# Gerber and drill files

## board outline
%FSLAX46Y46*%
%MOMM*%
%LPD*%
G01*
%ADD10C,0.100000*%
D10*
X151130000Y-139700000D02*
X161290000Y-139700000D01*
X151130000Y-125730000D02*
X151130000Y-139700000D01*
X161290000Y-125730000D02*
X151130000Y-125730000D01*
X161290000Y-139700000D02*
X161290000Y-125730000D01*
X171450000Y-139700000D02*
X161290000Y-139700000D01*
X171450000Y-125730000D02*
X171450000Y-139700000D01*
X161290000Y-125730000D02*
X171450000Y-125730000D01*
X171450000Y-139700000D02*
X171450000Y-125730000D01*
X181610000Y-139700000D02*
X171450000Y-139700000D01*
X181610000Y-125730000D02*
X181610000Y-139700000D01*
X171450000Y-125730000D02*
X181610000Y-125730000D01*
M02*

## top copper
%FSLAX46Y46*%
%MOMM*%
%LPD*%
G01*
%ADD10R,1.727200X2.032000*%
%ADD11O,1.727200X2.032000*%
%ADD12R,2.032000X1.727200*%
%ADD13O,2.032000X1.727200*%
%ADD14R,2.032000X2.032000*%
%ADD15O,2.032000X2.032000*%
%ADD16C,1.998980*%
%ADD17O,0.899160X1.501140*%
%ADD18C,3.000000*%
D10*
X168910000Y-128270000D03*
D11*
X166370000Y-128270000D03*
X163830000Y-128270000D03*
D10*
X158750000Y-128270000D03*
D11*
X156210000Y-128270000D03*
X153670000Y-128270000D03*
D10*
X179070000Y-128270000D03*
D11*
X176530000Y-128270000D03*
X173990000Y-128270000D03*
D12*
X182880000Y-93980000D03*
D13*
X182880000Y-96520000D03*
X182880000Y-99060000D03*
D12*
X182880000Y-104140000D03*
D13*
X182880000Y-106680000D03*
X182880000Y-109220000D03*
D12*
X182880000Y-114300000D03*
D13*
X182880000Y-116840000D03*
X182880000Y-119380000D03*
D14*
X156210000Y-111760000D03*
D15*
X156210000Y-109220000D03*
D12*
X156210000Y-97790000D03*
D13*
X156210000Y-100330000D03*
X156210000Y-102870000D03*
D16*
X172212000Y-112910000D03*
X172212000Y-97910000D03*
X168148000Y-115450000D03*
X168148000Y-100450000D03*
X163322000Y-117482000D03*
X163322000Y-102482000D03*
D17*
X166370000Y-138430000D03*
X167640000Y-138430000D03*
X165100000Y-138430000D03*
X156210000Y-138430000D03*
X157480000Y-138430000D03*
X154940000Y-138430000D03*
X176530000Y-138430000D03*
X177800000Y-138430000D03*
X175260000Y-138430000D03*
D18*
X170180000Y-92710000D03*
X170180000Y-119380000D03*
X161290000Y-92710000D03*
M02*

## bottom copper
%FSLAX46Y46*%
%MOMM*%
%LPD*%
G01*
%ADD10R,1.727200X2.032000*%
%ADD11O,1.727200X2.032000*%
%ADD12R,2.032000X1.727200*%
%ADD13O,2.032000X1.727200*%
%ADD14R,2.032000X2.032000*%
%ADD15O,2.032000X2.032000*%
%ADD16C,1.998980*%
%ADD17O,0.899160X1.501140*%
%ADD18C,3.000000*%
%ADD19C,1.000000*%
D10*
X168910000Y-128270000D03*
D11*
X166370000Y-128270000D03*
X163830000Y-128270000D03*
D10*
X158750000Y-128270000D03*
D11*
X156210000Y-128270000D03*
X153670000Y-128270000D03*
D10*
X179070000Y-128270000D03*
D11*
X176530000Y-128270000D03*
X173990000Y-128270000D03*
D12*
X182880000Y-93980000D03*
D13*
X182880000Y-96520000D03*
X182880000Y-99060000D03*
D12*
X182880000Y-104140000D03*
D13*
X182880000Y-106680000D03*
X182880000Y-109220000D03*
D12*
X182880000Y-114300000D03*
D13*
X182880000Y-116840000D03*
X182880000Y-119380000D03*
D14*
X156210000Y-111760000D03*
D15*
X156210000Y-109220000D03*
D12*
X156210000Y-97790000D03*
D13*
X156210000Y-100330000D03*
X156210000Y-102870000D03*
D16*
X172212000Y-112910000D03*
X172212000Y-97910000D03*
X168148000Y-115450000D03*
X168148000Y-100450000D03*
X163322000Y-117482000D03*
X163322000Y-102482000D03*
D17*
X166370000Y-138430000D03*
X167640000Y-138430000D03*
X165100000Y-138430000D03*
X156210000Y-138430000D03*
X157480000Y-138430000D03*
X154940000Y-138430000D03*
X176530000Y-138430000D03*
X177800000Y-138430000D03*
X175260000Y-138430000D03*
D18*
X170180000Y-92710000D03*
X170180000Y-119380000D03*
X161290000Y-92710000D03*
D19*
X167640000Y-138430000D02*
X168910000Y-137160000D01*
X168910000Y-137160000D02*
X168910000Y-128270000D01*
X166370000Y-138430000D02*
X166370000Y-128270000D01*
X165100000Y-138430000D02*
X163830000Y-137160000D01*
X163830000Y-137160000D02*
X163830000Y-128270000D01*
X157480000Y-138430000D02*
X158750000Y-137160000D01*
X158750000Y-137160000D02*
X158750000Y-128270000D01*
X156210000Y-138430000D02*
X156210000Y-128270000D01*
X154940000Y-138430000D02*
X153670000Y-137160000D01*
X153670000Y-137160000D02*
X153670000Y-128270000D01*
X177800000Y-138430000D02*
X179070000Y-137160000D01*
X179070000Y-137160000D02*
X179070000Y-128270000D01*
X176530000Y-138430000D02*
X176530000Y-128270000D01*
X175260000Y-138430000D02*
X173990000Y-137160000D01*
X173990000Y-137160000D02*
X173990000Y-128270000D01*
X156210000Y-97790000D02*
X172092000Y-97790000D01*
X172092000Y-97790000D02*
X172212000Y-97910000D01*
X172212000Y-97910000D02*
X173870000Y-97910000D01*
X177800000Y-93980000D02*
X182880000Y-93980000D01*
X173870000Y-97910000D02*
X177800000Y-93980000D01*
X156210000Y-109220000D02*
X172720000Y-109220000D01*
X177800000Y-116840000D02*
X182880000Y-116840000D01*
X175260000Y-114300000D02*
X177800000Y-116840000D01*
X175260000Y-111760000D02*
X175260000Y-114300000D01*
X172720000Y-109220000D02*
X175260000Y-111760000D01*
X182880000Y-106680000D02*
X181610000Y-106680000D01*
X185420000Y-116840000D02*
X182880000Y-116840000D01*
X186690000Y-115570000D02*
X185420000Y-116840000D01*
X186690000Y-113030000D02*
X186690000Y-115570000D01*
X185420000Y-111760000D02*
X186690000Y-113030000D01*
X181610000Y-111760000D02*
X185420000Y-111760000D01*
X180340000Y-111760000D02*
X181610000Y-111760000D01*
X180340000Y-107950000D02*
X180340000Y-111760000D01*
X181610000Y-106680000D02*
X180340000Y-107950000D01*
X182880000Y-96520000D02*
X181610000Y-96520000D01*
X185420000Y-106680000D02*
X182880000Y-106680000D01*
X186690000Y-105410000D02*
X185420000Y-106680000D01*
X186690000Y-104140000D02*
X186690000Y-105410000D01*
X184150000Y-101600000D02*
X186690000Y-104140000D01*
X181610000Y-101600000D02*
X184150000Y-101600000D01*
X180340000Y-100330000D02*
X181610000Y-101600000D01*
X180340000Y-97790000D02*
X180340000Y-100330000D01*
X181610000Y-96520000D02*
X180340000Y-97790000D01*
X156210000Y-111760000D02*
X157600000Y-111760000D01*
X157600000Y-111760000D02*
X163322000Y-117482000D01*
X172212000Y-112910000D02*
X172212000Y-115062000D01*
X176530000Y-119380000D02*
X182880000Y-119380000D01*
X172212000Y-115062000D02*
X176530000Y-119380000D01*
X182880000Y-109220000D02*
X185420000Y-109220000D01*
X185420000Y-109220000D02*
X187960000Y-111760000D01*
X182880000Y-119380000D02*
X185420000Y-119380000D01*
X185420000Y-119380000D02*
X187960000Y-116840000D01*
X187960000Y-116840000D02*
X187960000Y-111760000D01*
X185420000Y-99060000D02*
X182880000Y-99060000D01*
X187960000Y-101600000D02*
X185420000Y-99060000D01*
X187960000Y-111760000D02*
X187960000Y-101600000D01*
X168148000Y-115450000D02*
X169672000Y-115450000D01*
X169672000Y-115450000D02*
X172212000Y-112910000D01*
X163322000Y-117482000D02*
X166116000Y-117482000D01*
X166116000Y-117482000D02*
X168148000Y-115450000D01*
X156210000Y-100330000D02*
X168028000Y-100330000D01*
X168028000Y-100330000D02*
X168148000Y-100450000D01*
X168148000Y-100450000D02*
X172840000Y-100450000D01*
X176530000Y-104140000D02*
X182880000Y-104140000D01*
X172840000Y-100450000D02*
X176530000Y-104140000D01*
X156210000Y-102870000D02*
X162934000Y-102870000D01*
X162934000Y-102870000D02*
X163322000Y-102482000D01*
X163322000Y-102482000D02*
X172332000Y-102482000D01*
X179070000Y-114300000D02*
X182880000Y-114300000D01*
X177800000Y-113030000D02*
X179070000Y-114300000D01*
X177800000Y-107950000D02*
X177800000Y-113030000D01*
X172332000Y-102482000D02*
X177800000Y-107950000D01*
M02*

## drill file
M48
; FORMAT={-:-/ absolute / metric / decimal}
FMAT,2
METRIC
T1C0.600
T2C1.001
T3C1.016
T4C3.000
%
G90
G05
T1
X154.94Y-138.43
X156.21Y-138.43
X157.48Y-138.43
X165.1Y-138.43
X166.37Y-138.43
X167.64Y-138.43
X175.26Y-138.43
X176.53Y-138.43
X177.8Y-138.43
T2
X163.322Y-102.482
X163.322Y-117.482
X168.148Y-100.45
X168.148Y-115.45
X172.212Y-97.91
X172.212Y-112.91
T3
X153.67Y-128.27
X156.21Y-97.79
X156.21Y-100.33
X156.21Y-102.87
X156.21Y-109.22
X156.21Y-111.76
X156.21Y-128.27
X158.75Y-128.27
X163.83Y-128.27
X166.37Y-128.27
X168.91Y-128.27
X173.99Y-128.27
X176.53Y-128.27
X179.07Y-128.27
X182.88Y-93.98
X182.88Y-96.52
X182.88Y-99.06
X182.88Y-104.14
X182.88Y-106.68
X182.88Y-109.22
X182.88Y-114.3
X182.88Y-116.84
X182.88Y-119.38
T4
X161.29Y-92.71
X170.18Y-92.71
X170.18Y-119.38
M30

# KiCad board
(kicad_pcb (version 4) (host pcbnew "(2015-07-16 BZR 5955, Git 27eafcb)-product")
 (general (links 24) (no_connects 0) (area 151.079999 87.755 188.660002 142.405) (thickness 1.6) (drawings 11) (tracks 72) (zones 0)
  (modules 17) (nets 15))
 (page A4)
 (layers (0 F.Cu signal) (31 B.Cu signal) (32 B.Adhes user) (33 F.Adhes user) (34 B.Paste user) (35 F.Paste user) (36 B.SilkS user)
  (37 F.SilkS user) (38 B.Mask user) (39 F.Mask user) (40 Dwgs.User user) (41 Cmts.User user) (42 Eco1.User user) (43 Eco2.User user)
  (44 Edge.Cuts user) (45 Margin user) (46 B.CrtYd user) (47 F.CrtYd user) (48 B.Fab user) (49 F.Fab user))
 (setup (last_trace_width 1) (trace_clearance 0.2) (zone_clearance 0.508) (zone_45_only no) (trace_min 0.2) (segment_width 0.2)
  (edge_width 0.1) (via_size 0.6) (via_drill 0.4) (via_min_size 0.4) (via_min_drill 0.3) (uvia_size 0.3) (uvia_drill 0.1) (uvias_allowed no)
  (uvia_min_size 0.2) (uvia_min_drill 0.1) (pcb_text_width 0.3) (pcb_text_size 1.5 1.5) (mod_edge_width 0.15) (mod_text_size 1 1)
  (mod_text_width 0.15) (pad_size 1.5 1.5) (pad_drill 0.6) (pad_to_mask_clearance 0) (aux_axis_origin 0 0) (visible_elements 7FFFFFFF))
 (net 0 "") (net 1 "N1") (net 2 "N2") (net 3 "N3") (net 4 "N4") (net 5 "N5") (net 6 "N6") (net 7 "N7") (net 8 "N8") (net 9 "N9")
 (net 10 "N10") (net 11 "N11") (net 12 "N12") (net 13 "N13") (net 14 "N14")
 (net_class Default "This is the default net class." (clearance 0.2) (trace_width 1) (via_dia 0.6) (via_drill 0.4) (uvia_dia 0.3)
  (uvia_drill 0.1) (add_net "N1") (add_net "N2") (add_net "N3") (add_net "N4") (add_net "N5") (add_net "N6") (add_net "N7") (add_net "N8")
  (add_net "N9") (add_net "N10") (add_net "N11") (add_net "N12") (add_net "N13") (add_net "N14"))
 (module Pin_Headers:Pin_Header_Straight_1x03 (layer F.Cu) (at 168.91 128.27 270)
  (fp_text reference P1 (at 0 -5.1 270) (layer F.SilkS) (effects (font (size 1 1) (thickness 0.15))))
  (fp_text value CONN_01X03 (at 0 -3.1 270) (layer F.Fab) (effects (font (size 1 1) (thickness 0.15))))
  (pad 1 thru_hole rect (at 0 0 270) (size 2.032 1.7272) (drill 1.016) (layers *.Cu *.Mask F.SilkS) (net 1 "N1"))
  (pad 2 thru_hole oval (at 0 2.54 270) (size 2.032 1.7272) (drill 1.016) (layers *.Cu *.Mask F.SilkS) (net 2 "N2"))
  (pad 3 thru_hole oval (at 0 5.08 270) (size 2.032 1.7272) (drill 1.016) (layers *.Cu *.Mask F.SilkS) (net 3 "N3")))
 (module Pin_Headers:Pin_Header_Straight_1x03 (layer F.Cu) (at 158.75 128.27 270)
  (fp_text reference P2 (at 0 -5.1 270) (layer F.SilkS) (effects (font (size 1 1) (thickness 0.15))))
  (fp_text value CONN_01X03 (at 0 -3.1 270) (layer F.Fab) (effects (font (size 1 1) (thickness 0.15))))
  (pad 1 thru_hole rect (at 0 0 270) (size 2.032 1.7272) (drill 1.016) (layers *.Cu *.Mask F.SilkS) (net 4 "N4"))
  (pad 2 thru_hole oval (at 0 2.54 270) (size 2.032 1.7272) (drill 1.016) (layers *.Cu *.Mask F.SilkS) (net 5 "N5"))
  (pad 3 thru_hole oval (at 0 5.08 270) (size 2.032 1.7272) (drill 1.016) (layers *.Cu *.Mask F.SilkS) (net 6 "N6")))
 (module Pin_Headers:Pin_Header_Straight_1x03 (layer F.Cu) (at 179.07 128.27 270)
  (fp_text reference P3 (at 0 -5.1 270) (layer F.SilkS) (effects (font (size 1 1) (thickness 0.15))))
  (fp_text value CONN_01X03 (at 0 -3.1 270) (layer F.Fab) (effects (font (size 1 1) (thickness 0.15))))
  (pad 1 thru_hole rect (at 0 0 270) (size 2.032 1.7272) (drill 1.016) (layers *.Cu *.Mask F.SilkS) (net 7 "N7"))
  (pad 2 thru_hole oval (at 0 2.54 270) (size 2.032 1.7272) (drill 1.016) (layers *.Cu *.Mask F.SilkS) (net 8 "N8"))
  (pad 3 thru_hole oval (at 0 5.08 270) (size 2.032 1.7272) (drill 1.016) (layers *.Cu *.Mask F.SilkS) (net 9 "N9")))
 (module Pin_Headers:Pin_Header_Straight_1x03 (layer F.Cu) (at 182.88 93.98)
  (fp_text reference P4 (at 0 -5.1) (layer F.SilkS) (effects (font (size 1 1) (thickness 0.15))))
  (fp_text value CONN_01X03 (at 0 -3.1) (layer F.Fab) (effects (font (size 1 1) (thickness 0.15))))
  (pad 1 thru_hole rect (at 0 0) (size 2.032 1.7272) (drill 1.016) (layers *.Cu *.Mask F.SilkS) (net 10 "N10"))
  (pad 2 thru_hole oval (at 0 2.54) (size 2.032 1.7272) (drill 1.016) (layers *.Cu *.Mask F.SilkS) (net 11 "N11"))
  (pad 3 thru_hole oval (at 0 5.08) (size 2.032 1.7272) (drill 1.016) (layers *.Cu *.Mask F.SilkS) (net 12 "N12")))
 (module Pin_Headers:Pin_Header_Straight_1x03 (layer F.Cu) (at 182.88 104.14)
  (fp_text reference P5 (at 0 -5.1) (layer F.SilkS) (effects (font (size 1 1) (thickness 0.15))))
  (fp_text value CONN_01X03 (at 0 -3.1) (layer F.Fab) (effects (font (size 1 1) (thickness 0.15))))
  (pad 1 thru_hole rect (at 0 0) (size 2.032 1.7272) (drill 1.016) (layers *.Cu *.Mask F.SilkS) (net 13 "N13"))
  (pad 2 thru_hole oval (at 0 2.54) (size 2.032 1.7272) (drill 1.016) (layers *.Cu *.Mask F.SilkS) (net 11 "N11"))
  (pad 3 thru_hole oval (at 0 5.08) (size 2.032 1.7272) (drill 1.016) (layers *.Cu *.Mask F.SilkS) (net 12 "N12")))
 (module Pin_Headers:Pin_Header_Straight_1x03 (layer F.Cu) (at 182.88 114.3)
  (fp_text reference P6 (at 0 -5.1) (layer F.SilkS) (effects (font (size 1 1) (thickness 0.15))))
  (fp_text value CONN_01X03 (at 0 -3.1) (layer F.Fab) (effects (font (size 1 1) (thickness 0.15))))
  (pad 1 thru_hole rect (at 0 0) (size 2.032 1.7272) (drill 1.016) (layers *.Cu *.Mask F.SilkS) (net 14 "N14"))
  (pad 2 thru_hole oval (at 0 2.54) (size 2.032 1.7272) (drill 1.016) (layers *.Cu *.Mask F.SilkS) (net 11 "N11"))
  (pad 3 thru_hole oval (at 0 5.08) (size 2.032 1.7272) (drill 1.016) (layers *.Cu *.Mask F.SilkS) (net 12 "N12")))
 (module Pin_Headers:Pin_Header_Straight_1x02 (layer F.Cu) (at 156.21 111.76 180)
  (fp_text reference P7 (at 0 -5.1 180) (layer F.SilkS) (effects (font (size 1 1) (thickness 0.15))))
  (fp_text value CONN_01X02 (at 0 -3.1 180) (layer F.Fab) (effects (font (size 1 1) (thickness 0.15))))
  (pad 1 thru_hole rect (at 0 0 180) (size 2.032 2.032) (drill 1.016) (layers *.Cu *.Mask F.SilkS) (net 12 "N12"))
  (pad 2 thru_hole oval (at 0 2.54 180) (size 2.032 2.032) (drill 1.016) (layers *.Cu *.Mask F.SilkS) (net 11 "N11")))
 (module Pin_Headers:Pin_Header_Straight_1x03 (layer F.Cu) (at 156.21 97.79)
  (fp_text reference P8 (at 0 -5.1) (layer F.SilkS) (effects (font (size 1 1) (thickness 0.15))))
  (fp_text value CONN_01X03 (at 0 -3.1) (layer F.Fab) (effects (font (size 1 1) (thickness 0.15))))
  (pad 1 thru_hole rect (at 0 0) (size 2.032 1.7272) (drill 1.016) (layers *.Cu *.Mask F.SilkS) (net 10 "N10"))
  (pad 2 thru_hole oval (at 0 2.54) (size 2.032 1.7272) (drill 1.016) (layers *.Cu *.Mask F.SilkS) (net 13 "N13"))
  (pad 3 thru_hole oval (at 0 5.08) (size 2.032 1.7272) (drill 1.016) (layers *.Cu *.Mask F.SilkS) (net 14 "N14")))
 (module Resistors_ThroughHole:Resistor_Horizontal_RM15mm (layer F.Cu) (at 172.212 105.41 90)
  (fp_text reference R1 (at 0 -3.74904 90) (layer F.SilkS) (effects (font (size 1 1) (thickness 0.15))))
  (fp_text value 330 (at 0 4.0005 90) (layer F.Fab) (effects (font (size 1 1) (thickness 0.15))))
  (pad 1 thru_hole circle (at -7.5 0 90) (size 1.99898 1.99898) (drill 1.00076) (layers *.Cu *.SilkS *.Mask) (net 12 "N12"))
  (pad 2 thru_hole circle (at 7.5 0 90) (size 1.99898 1.99898) (drill 1.00076) (layers *.Cu *.SilkS *.Mask) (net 10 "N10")))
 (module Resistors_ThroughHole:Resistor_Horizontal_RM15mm (layer F.Cu) (at 168.148 107.95 90)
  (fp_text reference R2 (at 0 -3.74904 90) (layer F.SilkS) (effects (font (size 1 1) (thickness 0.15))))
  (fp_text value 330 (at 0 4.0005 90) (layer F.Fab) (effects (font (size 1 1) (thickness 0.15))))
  (pad 1 thru_hole circle (at -7.5 0 90) (size 1.99898 1.99898) (drill 1.00076) (layers *.Cu *.SilkS *.Mask) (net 12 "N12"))
  (pad 2 thru_hole circle (at 7.5 0 90) (size 1.99898 1.99898) (drill 1.00076) (layers *.Cu *.SilkS *.Mask) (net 13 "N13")))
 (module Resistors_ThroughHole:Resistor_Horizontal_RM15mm (layer F.Cu) (at 163.322 109.982 90)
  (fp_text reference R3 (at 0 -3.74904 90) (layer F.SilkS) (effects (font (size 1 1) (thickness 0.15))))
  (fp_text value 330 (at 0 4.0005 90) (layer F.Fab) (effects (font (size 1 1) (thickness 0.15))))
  (pad 1 thru_hole circle (at -7.5 0 90) (size 1.99898 1.99898) (drill 1.00076) (layers *.Cu *.SilkS *.Mask) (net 12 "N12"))
  (pad 2 thru_hole circle (at 7.5 0 90) (size 1.99898 1.99898) (drill 1.00076) (layers *.Cu *.SilkS *.Mask) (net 14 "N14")))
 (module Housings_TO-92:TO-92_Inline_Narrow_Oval (layer F.Cu) (at 165.1 138.43)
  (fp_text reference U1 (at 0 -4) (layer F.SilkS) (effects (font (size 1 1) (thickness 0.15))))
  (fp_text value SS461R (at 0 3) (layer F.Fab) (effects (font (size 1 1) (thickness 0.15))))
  (pad 2 thru_hole oval (at 1.27 0 180) (size 0.89916 1.50114) (drill 0.6) (layers *.Cu *.Mask F.SilkS) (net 2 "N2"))
  (pad 3 thru_hole oval (at 2.54 0 180) (size 0.89916 1.50114) (drill 0.6) (layers *.Cu *.Mask F.SilkS) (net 1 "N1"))
  (pad 1 thru_hole oval (at 0 0 180) (size 0.89916 1.50114) (drill 0.6) (layers *.Cu *.Mask F.SilkS) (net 3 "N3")))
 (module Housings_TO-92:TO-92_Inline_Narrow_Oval (layer F.Cu) (at 154.94 138.43)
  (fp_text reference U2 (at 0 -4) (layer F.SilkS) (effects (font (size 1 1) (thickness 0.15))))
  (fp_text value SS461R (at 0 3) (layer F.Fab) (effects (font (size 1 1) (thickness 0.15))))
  (pad 2 thru_hole oval (at 1.27 0 180) (size 0.89916 1.50114) (drill 0.6) (layers *.Cu *.Mask F.SilkS) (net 5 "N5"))
  (pad 3 thru_hole oval (at 2.54 0 180) (size 0.89916 1.50114) (drill 0.6) (layers *.Cu *.Mask F.SilkS) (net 4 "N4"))
  (pad 1 thru_hole oval (at 0 0 180) (size 0.89916 1.50114) (drill 0.6) (layers *.Cu *.Mask F.SilkS) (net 6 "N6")))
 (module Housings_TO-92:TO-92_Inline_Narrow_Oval (layer F.Cu) (at 175.26 138.43)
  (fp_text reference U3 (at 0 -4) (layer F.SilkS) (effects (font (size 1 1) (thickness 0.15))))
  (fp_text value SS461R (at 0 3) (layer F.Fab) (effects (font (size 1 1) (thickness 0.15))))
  (pad 2 thru_hole oval (at 1.27 0 180) (size 0.89916 1.50114) (drill 0.6) (layers *.Cu *.Mask F.SilkS) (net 8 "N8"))
  (pad 3 thru_hole oval (at 2.54 0 180) (size 0.89916 1.50114) (drill 0.6) (layers *.Cu *.Mask F.SilkS) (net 7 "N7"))
  (pad 1 thru_hole oval (at 0 0 180) (size 0.89916 1.50114) (drill 0.6) (layers *.Cu *.Mask F.SilkS) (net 9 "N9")))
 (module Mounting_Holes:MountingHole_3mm (layer F.Cu) (at 170.18 92.71)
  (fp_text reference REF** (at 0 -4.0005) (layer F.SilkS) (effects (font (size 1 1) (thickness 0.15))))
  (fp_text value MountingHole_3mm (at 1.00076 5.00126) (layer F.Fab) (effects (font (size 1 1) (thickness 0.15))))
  (pad 1 thru_hole circle (at 0 0) (size 3 3) (drill 3) (layers)))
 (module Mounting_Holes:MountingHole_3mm (layer F.Cu) (at 170.18 119.38)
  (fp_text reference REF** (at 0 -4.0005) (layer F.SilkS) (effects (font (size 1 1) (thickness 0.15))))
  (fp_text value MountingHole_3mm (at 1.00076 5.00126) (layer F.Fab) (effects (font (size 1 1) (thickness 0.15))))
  (pad 1 thru_hole circle (at 0 0) (size 3 3) (drill 3) (layers)))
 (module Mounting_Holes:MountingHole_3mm (layer F.Cu) (at 161.29 92.71)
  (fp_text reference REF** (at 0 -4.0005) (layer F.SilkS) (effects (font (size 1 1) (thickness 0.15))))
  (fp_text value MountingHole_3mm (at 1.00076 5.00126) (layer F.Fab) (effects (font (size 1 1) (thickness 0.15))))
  (pad 1 thru_hole circle (at 0 0) (size 3 3) (drill 3) (layers)))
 (gr_line (start 151.13 139.7) (end 161.29 139.7) (angle 90) (layer Edge.Cuts) (width 0.1))
 (gr_line (start 151.13 125.73) (end 151.13 139.7) (angle 90) (layer Edge.Cuts) (width 0.1))
 (gr_line (start 161.29 125.73) (end 151.13 125.73) (angle 90) (layer Edge.Cuts) (width 0.1))
 (gr_line (start 161.29 139.7) (end 161.29 125.73) (angle 90) (layer Edge.Cuts) (width 0.1))
 (gr_line (start 171.45 139.7) (end 161.29 139.7) (angle 90) (layer Edge.Cuts) (width 0.1))
 (gr_line (start 171.45 125.73) (end 171.45 139.7) (angle 90) (layer Edge.Cuts) (width 0.1))
 (gr_line (start 161.29 125.73) (end 171.45 125.73) (angle 90) (layer Edge.Cuts) (width 0.1))
 (gr_line (start 171.45 139.7) (end 171.45 125.73) (angle 90) (layer Edge.Cuts) (width 0.1))
 (gr_line (start 181.61 139.7) (end 171.45 139.7) (angle 90) (layer Edge.Cuts) (width 0.1))
 (gr_line (start 181.61 125.73) (end 181.61 139.7) (angle 90) (layer Edge.Cuts) (width 0.1))
 (gr_line (start 171.45 125.73) (end 181.61 125.73) (angle 90) (layer Edge.Cuts) (width 0.1))
 (segment (start 167.64 138.43) (end 168.91 137.16) (width 1) (layer B.Cu) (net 1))
 (segment (start 168.91 137.16) (end 168.91 128.27) (width 1) (layer B.Cu) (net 1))
 (segment (start 166.37 138.43) (end 166.37 128.27) (width 1) (layer B.Cu) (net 2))
 (segment (start 165.1 138.43) (end 163.83 137.16) (width 1) (layer B.Cu) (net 3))
 (segment (start 163.83 137.16) (end 163.83 128.27) (width 1) (layer B.Cu) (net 3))
 (segment (start 157.48 138.43) (end 158.75 137.16) (width 1) (layer B.Cu) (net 4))
 (segment (start 158.75 137.16) (end 158.75 128.27) (width 1) (layer B.Cu) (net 4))
 (segment (start 156.21 138.43) (end 156.21 128.27) (width 1) (layer B.Cu) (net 5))
 (segment (start 154.94 138.43) (end 153.67 137.16) (width 1) (layer B.Cu) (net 6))
 (segment (start 153.67 137.16) (end 153.67 128.27) (width 1) (layer B.Cu) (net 6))
 (segment (start 177.8 138.43) (end 179.07 137.16) (width 1) (layer B.Cu) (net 7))
 (segment (start 179.07 137.16) (end 179.07 128.27) (width 1) (layer B.Cu) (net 7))
 (segment (start 176.53 138.43) (end 176.53 128.27) (width 1) (layer B.Cu) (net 8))
 (segment (start 175.26 138.43) (end 173.99 137.16) (width 1) (layer B.Cu) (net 9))
 (segment (start 173.99 137.16) (end 173.99 128.27) (width 1) (layer B.Cu) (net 9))
 (segment (start 156.21 97.79) (end 172.092 97.79) (width 1) (layer B.Cu) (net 10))
 (segment (start 172.092 97.79) (end 172.212 97.91) (width 1) (layer B.Cu) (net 10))
 (segment (start 172.212 97.91) (end 173.87 97.91) (width 1) (layer B.Cu) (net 10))
 (segment (start 177.8 93.98) (end 182.88 93.98) (width 1) (layer B.Cu) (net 10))
 (segment (start 173.87 97.91) (end 177.8 93.98) (width 1) (layer B.Cu) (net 10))
 (segment (start 156.21 109.22) (end 172.72 109.22) (width 1) (layer B.Cu) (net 11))
 (segment (start 177.8 116.84) (end 182.88 116.84) (width 1) (layer B.Cu) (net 11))
 (segment (start 175.26 114.3) (end 177.8 116.84) (width 1) (layer B.Cu) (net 11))
 (segment (start 175.26 111.76) (end 175.26 114.3) (width 1) (layer B.Cu) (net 11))
 (segment (start 172.72 109.22) (end 175.26 111.76) (width 1) (layer B.Cu) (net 11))
 (segment (start 182.88 106.68) (end 181.61 106.68) (width 1) (layer B.Cu) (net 11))
 (segment (start 185.42 116.84) (end 182.88 116.84) (width 1) (layer B.Cu) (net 11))
 (segment (start 186.69 115.57) (end 185.42 116.84) (width 1) (layer B.Cu) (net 11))
 (segment (start 186.69 113.03) (end 186.69 115.57) (width 1) (layer B.Cu) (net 11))
 (segment (start 185.42 111.76) (end 186.69 113.03) (width 1) (layer B.Cu) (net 11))
 (segment (start 181.61 111.76) (end 185.42 111.76) (width 1) (layer B.Cu) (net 11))
 (segment (start 180.34 111.76) (end 181.61 111.76) (width 1) (layer B.Cu) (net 11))
 (segment (start 180.34 107.95) (end 180.34 111.76) (width 1) (layer B.Cu) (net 11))
 (segment (start 181.61 106.68) (end 180.34 107.95) (width 1) (layer B.Cu) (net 11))
 (segment (start 182.88 96.52) (end 181.61 96.52) (width 1) (layer B.Cu) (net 11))
 (segment (start 185.42 106.68) (end 182.88 106.68) (width 1) (layer B.Cu) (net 11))
 (segment (start 186.69 105.41) (end 185.42 106.68) (width 1) (layer B.Cu) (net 11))
 (segment (start 186.69 104.14) (end 186.69 105.41) (width 1) (layer B.Cu) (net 11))
 (segment (start 184.15 101.6) (end 186.69 104.14) (width 1) (layer B.Cu) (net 11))
 (segment (start 181.61 101.6) (end 184.15 101.6) (width 1) (layer B.Cu) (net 11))
 (segment (start 180.34 100.33) (end 181.61 101.6) (width 1) (layer B.Cu) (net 11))
 (segment (start 180.34 97.79) (end 180.34 100.33) (width 1) (layer B.Cu) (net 11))
 (segment (start 181.61 96.52) (end 180.34 97.79) (width 1) (layer B.Cu) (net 11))
 (segment (start 156.21 111.76) (end 157.6 111.76) (width 1) (layer B.Cu) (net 12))
 (segment (start 157.6 111.76) (end 163.322 117.482) (width 1) (layer B.Cu) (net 12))
 (segment (start 172.212 112.91) (end 172.212 115.062) (width 1) (layer B.Cu) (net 12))
 (segment (start 176.53 119.38) (end 182.88 119.38) (width 1) (layer B.Cu) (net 12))
 (segment (start 172.212 115.062) (end 176.53 119.38) (width 1) (layer B.Cu) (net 12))
 (segment (start 182.88 109.22) (end 185.42 109.22) (width 1) (layer B.Cu) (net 12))
 (segment (start 185.42 109.22) (end 187.96 111.76) (width 1) (layer B.Cu) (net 12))
 (segment (start 182.88 119.38) (end 185.42 119.38) (width 1) (layer B.Cu) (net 12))
 (segment (start 185.42 119.38) (end 187.96 116.84) (width 1) (layer B.Cu) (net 12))
 (segment (start 187.96 116.84) (end 187.96 111.76) (width 1) (layer B.Cu) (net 12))
 (segment (start 185.42 99.06) (end 182.88 99.06) (width 1) (layer B.Cu) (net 12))
 (segment (start 187.96 101.6) (end 185.42 99.06) (width 1) (layer B.Cu) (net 12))
 (segment (start 187.96 111.76) (end 187.96 101.6) (width 1) (layer B.Cu) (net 12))
 (segment (start 168.148 115.45) (end 169.672 115.45) (width 1) (layer B.Cu) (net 12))
 (segment (start 169.672 115.45) (end 172.212 112.91) (width 1) (layer B.Cu) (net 12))
 (segment (start 163.322 117.482) (end 166.116 117.482) (width 1) (layer B.Cu) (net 12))
 (segment (start 166.116 117.482) (end 168.148 115.45) (width 1) (layer B.Cu) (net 12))
 (segment (start 156.21 100.33) (end 168.028 100.33) (width 1) (layer B.Cu) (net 13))
 (segment (start 168.028 100.33) (end 168.148 100.45) (width 1) (layer B.Cu) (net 13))
 (segment (start 168.148 100.45) (end 172.84 100.45) (width 1) (layer B.Cu) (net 13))
 (segment (start 176.53 104.14) (end 182.88 104.14) (width 1) (layer B.Cu) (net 13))
 (segment (start 172.84 100.45) (end 176.53 104.14) (width 1) (layer B.Cu) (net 13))
 (segment (start 156.21 102.87) (end 162.934 102.87) (width 1) (layer B.Cu) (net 14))
 (segment (start 162.934 102.87) (end 163.322 102.482) (width 1) (layer B.Cu) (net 14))
 (segment (start 163.322 102.482) (end 172.332 102.482) (width 1) (layer B.Cu) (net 14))
 (segment (start 179.07 114.3) (end 182.88 114.3) (width 1) (layer B.Cu) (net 14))
 (segment (start 177.8 113.03) (end 179.07 114.3) (width 1) (layer B.Cu) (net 14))
 (segment (start 177.8 107.95) (end 177.8 113.03) (width 1) (layer B.Cu) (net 14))
 (segment (start 172.332 102.482) (end 177.8 107.95) (width 1) (layer B.Cu) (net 14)))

